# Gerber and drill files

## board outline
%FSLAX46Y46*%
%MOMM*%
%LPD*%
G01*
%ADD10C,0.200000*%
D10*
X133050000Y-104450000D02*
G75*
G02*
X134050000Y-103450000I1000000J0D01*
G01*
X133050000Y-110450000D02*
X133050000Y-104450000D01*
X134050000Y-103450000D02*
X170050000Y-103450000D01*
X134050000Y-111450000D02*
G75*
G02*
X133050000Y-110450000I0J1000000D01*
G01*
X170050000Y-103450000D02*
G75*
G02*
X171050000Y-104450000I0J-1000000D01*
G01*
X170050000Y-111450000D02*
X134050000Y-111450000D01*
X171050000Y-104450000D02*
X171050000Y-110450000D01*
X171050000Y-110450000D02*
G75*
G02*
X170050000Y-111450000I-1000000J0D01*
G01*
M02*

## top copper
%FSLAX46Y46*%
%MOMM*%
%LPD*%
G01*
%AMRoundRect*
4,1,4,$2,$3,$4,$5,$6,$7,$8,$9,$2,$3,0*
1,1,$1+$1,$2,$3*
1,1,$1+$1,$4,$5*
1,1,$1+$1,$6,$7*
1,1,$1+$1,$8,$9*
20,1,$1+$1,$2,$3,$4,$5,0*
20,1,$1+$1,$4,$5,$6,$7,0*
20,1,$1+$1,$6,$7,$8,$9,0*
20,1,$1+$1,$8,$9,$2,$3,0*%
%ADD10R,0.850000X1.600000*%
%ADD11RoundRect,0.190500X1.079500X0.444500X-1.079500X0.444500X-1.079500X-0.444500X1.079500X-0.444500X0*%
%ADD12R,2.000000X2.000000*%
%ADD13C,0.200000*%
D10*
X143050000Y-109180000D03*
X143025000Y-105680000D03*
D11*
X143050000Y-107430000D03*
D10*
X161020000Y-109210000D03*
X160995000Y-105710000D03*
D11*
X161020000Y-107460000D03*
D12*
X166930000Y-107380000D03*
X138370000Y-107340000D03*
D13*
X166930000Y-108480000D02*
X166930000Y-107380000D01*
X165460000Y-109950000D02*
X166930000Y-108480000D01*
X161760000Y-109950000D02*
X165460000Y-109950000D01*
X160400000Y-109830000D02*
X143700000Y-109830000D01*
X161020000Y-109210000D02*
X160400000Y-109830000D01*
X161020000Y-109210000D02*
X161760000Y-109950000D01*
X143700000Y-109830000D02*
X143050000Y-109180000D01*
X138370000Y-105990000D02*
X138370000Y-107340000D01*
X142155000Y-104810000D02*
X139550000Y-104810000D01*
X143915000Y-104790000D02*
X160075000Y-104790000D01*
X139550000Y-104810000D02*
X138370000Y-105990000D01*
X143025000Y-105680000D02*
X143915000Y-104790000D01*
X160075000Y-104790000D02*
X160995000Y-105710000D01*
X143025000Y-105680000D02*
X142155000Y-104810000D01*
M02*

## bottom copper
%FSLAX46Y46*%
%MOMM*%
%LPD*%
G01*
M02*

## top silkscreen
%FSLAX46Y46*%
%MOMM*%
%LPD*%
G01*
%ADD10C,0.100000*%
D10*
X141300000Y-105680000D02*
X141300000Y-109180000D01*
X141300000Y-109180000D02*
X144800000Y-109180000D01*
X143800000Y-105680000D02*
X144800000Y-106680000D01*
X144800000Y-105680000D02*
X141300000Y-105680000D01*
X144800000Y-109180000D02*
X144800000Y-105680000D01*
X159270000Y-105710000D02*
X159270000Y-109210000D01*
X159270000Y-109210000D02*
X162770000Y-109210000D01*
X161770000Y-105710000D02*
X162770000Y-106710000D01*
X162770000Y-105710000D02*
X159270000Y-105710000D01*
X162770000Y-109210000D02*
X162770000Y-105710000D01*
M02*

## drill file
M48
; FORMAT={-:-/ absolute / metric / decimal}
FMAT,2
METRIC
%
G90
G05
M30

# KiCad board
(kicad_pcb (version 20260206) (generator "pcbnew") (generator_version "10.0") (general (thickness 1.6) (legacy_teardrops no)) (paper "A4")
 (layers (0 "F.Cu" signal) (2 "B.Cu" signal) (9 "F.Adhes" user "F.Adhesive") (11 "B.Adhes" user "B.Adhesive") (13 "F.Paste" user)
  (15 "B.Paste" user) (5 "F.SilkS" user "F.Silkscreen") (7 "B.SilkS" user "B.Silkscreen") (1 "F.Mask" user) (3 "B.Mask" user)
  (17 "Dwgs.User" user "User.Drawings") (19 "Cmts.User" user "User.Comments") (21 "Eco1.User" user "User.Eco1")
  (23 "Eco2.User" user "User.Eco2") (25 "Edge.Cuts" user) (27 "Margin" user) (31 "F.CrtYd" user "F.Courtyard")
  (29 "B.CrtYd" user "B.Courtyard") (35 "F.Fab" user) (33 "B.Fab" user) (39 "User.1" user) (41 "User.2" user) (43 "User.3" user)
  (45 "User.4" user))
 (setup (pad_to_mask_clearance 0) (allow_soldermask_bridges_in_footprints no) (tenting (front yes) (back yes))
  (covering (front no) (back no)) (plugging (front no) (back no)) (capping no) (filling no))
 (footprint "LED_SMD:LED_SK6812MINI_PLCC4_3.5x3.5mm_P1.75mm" (layer "F.Cu") (at 143.05 107.43 90)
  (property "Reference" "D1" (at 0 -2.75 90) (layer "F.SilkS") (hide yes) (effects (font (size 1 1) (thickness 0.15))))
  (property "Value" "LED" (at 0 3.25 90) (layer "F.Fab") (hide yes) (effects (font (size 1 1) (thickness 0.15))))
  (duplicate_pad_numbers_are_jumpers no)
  (fp_line (start 1.75 -1.75) (end -1.75 -1.75) (stroke (width 0.1) (type solid)) (layer "F.SilkS"))
  (fp_line (start -1.75 -1.75) (end -1.75 1.75) (stroke (width 0.1) (type solid)) (layer "F.SilkS"))
  (fp_line (start 1.75 0.75) (end 0.75 1.75) (stroke (width 0.1) (type solid)) (layer "F.SilkS"))
  (fp_line (start 1.75 1.75) (end 1.75 -1.75) (stroke (width 0.1) (type solid)) (layer "F.SilkS"))
  (fp_line (start -1.75 1.75) (end 1.75 1.75) (stroke (width 0.1) (type solid)) (layer "F.SilkS"))
  (pad "1" smd rect (at -1.75 0 90) (size 1.6 0.85) (layers "F.Cu" "F.Mask" "F.Paste") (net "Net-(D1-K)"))
  (pad "2" smd rect (at 1.75 -0.025 90) (size 1.6 0.85) (layers "F.Cu" "F.Mask" "F.Paste") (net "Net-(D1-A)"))
  (pad "3" smd roundrect (at 0 0 180) (size 2.54 1.27) (layers "F.Cu" "F.Mask" "F.Paste") (roundrect_rratio 0.15)))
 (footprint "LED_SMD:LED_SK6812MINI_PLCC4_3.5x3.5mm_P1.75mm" (layer "F.Cu") (at 161.02 107.46 90)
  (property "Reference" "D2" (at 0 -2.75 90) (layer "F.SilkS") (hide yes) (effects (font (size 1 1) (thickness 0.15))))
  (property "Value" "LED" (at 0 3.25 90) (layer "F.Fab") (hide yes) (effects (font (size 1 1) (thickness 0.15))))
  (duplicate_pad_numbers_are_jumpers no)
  (fp_line (start 1.75 -1.75) (end -1.75 -1.75) (stroke (width 0.1) (type solid)) (layer "F.SilkS"))
  (fp_line (start -1.75 -1.75) (end -1.75 1.75) (stroke (width 0.1) (type solid)) (layer "F.SilkS"))
  (fp_line (start 1.75 0.75) (end 0.75 1.75) (stroke (width 0.1) (type solid)) (layer "F.SilkS"))
  (fp_line (start 1.75 1.75) (end 1.75 -1.75) (stroke (width 0.1) (type solid)) (layer "F.SilkS"))
  (fp_line (start -1.75 1.75) (end 1.75 1.75) (stroke (width 0.1) (type solid)) (layer "F.SilkS"))
  (pad "1" smd rect (at -1.75 0 90) (size 1.6 0.85) (layers "F.Cu" "F.Mask" "F.Paste") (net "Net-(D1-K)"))
  (pad "2" smd rect (at 1.75 -0.025 90) (size 1.6 0.85) (layers "F.Cu" "F.Mask" "F.Paste") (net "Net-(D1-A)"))
  (pad "3" smd roundrect (at 0 0 180) (size 2.54 1.27) (layers "F.Cu" "F.Mask" "F.Paste") (roundrect_rratio 0.15)))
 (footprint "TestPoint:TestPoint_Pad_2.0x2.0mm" (layer "F.Cu") (at 166.93 107.38)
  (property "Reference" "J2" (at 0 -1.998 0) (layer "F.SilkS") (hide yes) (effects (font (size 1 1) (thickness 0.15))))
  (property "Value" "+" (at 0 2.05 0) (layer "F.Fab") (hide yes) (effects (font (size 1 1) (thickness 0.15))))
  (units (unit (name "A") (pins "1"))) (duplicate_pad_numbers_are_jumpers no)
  (pad "1" smd rect (at 0 0) (size 2 2) (layers "F.Cu" "F.Mask") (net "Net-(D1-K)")))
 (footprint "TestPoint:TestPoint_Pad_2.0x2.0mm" (layer "F.Cu") (at 138.37 107.34)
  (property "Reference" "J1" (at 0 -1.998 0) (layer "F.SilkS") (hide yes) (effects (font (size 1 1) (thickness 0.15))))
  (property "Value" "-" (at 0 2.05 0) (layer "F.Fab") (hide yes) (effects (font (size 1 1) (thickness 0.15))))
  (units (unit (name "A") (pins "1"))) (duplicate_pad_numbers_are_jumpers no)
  (pad "1" smd rect (at 0 0) (size 2 2) (layers "F.Cu" "F.Mask") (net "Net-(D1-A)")))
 (gr_arc (start 133.05 104.45) (mid 133.342893 103.742893) (end 134.05 103.45) (stroke (width 0.2) (type solid)) (layer "Edge.Cuts"))
 (gr_line (start 133.05 110.45) (end 133.05 104.45) (stroke (width 0.2) (type solid)) (layer "Edge.Cuts"))
 (gr_line (start 134.05 103.45) (end 170.05 103.45) (stroke (width 0.2) (type solid)) (layer "Edge.Cuts"))
 (gr_arc (start 134.05 111.45) (mid 133.342893 111.157107) (end 133.05 110.45) (stroke (width 0.2) (type solid)) (layer "Edge.Cuts"))
 (gr_arc (start 170.05 103.45) (mid 170.757107 103.742893) (end 171.05 104.45) (stroke (width 0.2) (type solid)) (layer "Edge.Cuts"))
 (gr_line (start 170.05 111.45) (end 134.05 111.45) (stroke (width 0.2) (type solid)) (layer "Edge.Cuts"))
 (gr_line (start 171.05 104.45) (end 171.05 110.45) (stroke (width 0.2) (type solid)) (layer "Edge.Cuts"))
 (gr_arc (start 171.05 110.45) (mid 170.757107 111.157107) (end 170.05 111.45) (stroke (width 0.2) (type solid)) (layer "Edge.Cuts"))
 (segment (start 166.93 108.48) (end 166.93 107.38) (width 0.2) (layer "F.Cu") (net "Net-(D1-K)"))
 (segment (start 165.46 109.95) (end 166.93 108.48) (width 0.2) (layer "F.Cu") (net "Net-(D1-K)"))
 (segment (start 161.76 109.95) (end 165.46 109.95) (width 0.2) (layer "F.Cu") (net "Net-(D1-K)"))
 (segment (start 160.4 109.83) (end 143.7 109.83) (width 0.2) (layer "F.Cu") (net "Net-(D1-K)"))
 (segment (start 161.02 109.21) (end 160.4 109.83) (width 0.2) (layer "F.Cu") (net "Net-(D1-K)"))
 (segment (start 161.02 109.21) (end 161.76 109.95) (width 0.2) (layer "F.Cu") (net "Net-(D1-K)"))
 (segment (start 143.7 109.83) (end 143.05 109.18) (width 0.2) (layer "F.Cu") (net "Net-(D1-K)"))
 (segment (start 138.37 105.99) (end 138.37 107.34) (width 0.2) (layer "F.Cu") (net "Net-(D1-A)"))
 (segment (start 142.155 104.81) (end 139.55 104.81) (width 0.2) (layer "F.Cu") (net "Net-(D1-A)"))
 (segment (start 143.915 104.79) (end 160.075 104.79) (width 0.2) (layer "F.Cu") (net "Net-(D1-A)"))
 (segment (start 139.55 104.81) (end 138.37 105.99) (width 0.2) (layer "F.Cu") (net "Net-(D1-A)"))
 (segment (start 143.025 105.68) (end 143.915 104.79) (width 0.2) (layer "F.Cu") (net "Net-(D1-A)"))
 (segment (start 160.075 104.79) (end 160.995 105.71) (width 0.2) (layer "F.Cu") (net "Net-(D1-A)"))
 (segment (start 143.025 105.68) (end 142.155 104.81) (width 0.2) (layer "F.Cu") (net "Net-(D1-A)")))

